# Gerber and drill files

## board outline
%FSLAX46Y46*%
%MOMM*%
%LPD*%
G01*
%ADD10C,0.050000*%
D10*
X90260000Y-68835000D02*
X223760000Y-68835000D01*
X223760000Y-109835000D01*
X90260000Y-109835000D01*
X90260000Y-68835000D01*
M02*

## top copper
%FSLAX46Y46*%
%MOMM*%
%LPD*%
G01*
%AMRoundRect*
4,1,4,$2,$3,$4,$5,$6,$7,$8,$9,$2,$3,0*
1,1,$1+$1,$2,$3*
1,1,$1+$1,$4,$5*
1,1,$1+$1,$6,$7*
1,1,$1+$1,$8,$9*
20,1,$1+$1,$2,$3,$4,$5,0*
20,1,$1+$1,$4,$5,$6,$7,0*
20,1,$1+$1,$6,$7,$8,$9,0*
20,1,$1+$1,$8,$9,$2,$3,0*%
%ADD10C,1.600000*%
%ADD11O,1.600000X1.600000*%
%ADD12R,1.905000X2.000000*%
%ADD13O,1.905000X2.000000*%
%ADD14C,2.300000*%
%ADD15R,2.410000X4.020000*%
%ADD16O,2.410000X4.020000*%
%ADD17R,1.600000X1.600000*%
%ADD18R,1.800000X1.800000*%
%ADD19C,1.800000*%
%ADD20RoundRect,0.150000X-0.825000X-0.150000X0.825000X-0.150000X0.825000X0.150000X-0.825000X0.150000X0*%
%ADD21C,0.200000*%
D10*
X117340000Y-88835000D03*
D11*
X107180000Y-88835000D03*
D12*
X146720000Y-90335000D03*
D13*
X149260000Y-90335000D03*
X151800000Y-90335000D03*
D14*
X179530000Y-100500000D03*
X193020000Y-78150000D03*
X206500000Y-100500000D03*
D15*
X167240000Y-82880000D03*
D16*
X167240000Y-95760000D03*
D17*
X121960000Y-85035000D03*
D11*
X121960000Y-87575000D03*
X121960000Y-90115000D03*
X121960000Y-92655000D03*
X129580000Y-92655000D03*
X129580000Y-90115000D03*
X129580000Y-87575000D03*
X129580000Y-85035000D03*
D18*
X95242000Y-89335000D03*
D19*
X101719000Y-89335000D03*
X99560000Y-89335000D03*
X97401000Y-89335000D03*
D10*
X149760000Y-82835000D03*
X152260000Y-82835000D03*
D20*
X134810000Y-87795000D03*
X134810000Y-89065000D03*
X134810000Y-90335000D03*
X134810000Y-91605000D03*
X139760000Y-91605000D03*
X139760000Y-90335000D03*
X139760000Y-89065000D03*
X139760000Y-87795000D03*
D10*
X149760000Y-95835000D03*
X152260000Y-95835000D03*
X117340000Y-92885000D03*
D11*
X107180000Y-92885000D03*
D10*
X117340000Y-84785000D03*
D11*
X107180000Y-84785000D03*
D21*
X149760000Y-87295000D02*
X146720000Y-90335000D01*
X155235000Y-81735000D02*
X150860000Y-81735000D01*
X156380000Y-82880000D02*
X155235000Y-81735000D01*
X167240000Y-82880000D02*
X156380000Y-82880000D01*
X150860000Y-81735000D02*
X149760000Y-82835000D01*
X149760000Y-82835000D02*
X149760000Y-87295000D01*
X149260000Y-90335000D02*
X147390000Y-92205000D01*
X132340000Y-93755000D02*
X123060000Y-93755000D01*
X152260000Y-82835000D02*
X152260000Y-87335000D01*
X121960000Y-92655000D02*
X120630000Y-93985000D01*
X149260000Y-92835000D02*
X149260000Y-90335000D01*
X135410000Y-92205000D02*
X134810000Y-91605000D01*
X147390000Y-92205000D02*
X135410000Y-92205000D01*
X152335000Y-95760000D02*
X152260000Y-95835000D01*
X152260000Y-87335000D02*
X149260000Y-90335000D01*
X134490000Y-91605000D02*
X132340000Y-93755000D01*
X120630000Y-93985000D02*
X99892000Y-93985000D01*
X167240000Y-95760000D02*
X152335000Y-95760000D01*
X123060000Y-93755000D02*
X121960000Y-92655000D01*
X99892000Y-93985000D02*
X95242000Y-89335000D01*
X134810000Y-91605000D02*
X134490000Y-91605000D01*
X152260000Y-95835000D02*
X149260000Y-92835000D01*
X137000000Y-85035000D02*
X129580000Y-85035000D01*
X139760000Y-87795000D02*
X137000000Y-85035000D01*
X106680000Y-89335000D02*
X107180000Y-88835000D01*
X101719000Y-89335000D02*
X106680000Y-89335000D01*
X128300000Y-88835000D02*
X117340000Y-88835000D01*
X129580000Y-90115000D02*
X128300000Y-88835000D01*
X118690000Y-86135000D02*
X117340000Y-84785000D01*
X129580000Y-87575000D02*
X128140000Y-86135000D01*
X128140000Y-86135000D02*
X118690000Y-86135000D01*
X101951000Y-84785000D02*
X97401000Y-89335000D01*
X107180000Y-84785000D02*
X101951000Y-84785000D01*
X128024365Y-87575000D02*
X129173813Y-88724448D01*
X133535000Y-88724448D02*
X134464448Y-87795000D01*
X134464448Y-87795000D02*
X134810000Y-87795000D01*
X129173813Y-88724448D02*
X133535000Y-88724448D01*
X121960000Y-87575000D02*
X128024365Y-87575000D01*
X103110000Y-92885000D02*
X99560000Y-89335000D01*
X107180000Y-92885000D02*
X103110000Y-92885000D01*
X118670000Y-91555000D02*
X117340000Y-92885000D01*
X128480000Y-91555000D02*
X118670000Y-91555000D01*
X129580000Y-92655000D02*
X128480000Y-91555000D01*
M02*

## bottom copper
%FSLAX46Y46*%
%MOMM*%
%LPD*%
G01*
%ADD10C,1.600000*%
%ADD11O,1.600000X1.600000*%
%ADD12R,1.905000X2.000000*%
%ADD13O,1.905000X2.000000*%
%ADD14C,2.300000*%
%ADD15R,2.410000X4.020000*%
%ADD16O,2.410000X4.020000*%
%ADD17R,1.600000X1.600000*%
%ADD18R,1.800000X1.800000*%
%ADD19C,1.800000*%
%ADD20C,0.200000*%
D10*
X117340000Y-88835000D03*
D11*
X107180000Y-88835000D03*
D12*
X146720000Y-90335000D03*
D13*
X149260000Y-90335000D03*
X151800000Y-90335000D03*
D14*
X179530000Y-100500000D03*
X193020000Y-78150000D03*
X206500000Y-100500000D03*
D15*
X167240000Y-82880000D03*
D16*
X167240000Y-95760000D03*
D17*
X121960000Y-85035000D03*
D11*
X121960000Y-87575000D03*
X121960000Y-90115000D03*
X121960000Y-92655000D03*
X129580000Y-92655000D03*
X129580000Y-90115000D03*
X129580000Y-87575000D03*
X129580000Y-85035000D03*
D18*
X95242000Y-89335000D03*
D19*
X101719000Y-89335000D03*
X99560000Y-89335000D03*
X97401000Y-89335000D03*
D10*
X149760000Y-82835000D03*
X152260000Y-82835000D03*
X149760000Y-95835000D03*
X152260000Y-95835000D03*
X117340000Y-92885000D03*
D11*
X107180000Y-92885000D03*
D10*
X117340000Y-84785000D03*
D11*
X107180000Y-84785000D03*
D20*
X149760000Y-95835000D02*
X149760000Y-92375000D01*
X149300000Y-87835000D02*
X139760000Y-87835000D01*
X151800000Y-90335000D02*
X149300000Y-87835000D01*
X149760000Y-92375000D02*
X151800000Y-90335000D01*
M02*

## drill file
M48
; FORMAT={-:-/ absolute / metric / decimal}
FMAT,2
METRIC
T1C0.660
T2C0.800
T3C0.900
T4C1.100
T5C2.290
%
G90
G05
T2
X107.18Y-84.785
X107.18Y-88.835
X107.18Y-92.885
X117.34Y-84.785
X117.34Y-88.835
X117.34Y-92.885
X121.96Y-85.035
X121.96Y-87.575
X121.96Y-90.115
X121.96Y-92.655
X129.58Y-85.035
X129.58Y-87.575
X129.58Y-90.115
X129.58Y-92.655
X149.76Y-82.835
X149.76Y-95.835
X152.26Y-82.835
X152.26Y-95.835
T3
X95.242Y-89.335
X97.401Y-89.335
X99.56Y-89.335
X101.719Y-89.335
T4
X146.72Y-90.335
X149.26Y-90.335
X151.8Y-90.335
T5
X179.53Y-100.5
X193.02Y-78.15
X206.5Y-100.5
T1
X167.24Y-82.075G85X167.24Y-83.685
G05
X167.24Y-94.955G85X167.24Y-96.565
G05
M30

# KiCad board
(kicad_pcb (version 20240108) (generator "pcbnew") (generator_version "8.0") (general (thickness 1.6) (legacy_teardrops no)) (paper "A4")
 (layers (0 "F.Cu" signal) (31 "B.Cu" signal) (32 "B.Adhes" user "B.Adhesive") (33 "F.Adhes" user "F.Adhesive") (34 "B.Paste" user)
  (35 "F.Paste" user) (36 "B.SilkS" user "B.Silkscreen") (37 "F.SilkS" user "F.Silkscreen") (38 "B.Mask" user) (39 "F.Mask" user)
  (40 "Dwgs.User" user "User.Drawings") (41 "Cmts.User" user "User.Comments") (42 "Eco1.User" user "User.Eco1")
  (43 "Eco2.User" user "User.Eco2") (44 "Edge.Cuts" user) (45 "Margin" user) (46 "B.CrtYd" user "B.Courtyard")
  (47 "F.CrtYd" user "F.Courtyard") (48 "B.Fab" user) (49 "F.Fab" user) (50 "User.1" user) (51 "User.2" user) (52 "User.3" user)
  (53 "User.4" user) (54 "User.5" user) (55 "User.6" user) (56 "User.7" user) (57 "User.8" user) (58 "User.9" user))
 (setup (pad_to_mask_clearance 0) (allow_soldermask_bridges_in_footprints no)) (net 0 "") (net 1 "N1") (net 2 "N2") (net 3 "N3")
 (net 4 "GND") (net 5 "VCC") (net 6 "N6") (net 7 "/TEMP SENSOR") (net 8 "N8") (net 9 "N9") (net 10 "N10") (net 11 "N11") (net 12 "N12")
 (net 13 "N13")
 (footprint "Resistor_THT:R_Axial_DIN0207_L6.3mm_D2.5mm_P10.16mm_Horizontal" (layer "F.Cu") (at 117.34 88.835 180)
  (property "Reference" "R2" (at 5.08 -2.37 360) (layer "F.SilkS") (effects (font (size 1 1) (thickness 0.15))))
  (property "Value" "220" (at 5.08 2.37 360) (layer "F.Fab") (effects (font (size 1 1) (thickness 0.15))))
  (pad "1" thru_hole circle (at 0 0 180) (size 1.6 1.6) (drill 0.8) (layers "*.Cu" "*.Mask") (remove_unused_layers no) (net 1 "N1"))
  (pad "2" thru_hole oval (at 10.16 0 180) (size 1.6 1.6) (drill 0.8) (layers "*.Cu" "*.Mask") (remove_unused_layers no) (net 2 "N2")))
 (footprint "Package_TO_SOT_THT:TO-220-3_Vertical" (layer "F.Cu") (at 146.72 90.335)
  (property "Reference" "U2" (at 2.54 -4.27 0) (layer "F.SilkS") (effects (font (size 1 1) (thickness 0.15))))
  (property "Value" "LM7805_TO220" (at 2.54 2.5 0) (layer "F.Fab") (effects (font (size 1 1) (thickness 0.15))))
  (pad "1" thru_hole rect (at 0 0) (size 1.905 2) (drill 1.1) (layers "*.Cu" "*.Mask") (remove_unused_layers no) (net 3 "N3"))
  (pad "2" thru_hole oval (at 2.54 0) (size 1.905 2) (drill 1.1) (layers "*.Cu" "*.Mask") (remove_unused_layers no) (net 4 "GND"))
  (pad "3" thru_hole oval (at 5.08 0) (size 1.905 2) (drill 1.1) (layers "*.Cu" "*.Mask") (remove_unused_layers no) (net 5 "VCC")))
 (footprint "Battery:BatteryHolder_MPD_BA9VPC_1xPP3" (layer "F.Cu") (at 167.24 82.88)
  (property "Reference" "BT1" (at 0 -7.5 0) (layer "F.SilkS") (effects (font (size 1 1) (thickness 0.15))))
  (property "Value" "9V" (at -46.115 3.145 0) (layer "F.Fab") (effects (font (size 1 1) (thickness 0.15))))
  (pad "" np_thru_hole circle (at 12.29 17.62) (size 2.3 2.3) (drill 2.29) (layers "*.Cu" "*.Mask"))
  (pad "" np_thru_hole circle (at 25.78 -4.73) (size 2.3 2.3) (drill 2.29) (layers "*.Cu" "*.Mask"))
  (pad "" np_thru_hole circle (at 39.26 17.62) (size 2.3 2.3) (drill 2.29) (layers "*.Cu" "*.Mask"))
  (pad "1" thru_hole rect (at 0 0) (size 2.41 4.02) (drill oval 0.66 2.27) (layers "*.Cu" "*.Mask") (remove_unused_layers no) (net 3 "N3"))
  (pad "2" thru_hole oval (at 0 12.88) (size 2.41 4.02) (drill oval 0.66 2.27) (layers "*.Cu" "*.Mask") (remove_unused_layers no)
   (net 4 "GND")))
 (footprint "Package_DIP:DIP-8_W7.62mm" (layer "F.Cu") (at 121.96 85.035)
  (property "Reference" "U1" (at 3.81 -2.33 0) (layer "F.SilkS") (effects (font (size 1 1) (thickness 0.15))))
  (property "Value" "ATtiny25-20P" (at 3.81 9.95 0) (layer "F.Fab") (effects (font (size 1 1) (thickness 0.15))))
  (pad "1" thru_hole rect (at 0 0) (size 1.6 1.6) (drill 0.8) (layers "*.Cu" "*.Mask") (remove_unused_layers no) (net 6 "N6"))
  (pad "2" thru_hole oval (at 0 2.54) (size 1.6 1.6) (drill 0.8) (layers "*.Cu" "*.Mask") (remove_unused_layers no) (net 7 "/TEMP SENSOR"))
  (pad "3" thru_hole oval (at 0 5.08) (size 1.6 1.6) (drill 0.8) (layers "*.Cu" "*.Mask") (remove_unused_layers no) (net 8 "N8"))
  (pad "4" thru_hole oval (at 0 7.62) (size 1.6 1.6) (drill 0.8) (layers "*.Cu" "*.Mask") (remove_unused_layers no) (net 4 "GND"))
  (pad "5" thru_hole oval (at 7.62 7.62) (size 1.6 1.6) (drill 0.8) (layers "*.Cu" "*.Mask") (remove_unused_layers no) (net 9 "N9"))
  (pad "6" thru_hole oval (at 7.62 5.08) (size 1.6 1.6) (drill 0.8) (layers "*.Cu" "*.Mask") (remove_unused_layers no) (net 1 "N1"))
  (pad "7" thru_hole oval (at 7.62 2.54) (size 1.6 1.6) (drill 0.8) (layers "*.Cu" "*.Mask") (remove_unused_layers no) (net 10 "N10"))
  (pad "8" thru_hole oval (at 7.62 0) (size 1.6 1.6) (drill 0.8) (layers "*.Cu" "*.Mask") (remove_unused_layers no) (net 5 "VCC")))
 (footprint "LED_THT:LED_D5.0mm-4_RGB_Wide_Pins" (layer "F.Cu") (at 95.242 89.335)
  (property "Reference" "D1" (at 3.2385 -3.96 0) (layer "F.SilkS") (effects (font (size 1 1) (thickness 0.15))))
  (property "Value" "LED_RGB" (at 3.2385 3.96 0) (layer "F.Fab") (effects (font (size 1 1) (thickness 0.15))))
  (pad "1" thru_hole rect (at 0 0) (size 1.8 1.8) (drill 0.9) (layers "*.Cu" "*.Mask") (remove_unused_layers no) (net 4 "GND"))
  (pad "4" thru_hole circle (at 6.477 0) (size 1.8 1.8) (drill 0.9) (layers "*.Cu" "*.Mask") (remove_unused_layers no) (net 2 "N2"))
  (pad "5" thru_hole circle (at 4.318 0) (size 1.8 1.8) (drill 0.9) (layers "*.Cu" "*.Mask") (remove_unused_layers no) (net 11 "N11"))
  (pad "6" thru_hole circle (at 2.159 0) (size 1.8 1.8) (drill 0.9) (layers "*.Cu" "*.Mask") (remove_unused_layers no) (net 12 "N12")))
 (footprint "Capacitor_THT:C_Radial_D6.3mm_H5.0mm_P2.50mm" (layer "F.Cu") (at 149.76 82.835)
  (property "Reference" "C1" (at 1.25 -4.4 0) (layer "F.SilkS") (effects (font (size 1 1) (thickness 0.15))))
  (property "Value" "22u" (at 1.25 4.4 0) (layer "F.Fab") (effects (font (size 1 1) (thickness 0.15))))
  (pad "1" thru_hole circle (at 0 0) (size 1.6 1.6) (drill 0.8) (layers "*.Cu" "*.Mask") (remove_unused_layers no) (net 3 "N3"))
  (pad "2" thru_hole circle (at 2.5 0) (size 1.6 1.6) (drill 0.8) (layers "*.Cu" "*.Mask") (remove_unused_layers no) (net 4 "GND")))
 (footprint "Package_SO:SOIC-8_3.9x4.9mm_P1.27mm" (layer "F.Cu") (at 137.285 89.7)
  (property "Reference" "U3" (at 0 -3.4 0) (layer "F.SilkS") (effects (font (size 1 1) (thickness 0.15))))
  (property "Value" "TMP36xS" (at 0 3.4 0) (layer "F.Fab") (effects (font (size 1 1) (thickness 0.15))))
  (pad "1" smd roundrect (at -2.475 -1.905) (size 1.95 0.6) (layers "F.Cu" "F.Paste" "F.Mask") (roundrect_rratio 0.25)
   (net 7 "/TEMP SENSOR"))
  (pad "2" smd roundrect (at -2.475 -0.635) (size 1.95 0.6) (layers "F.Cu" "F.Paste" "F.Mask") (roundrect_rratio 0.25))
  (pad "3" smd roundrect (at -2.475 0.635) (size 1.95 0.6) (layers "F.Cu" "F.Paste" "F.Mask") (roundrect_rratio 0.25))
  (pad "4" smd roundrect (at -2.475 1.905) (size 1.95 0.6) (layers "F.Cu" "F.Paste" "F.Mask") (roundrect_rratio 0.25) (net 4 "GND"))
  (pad "5" smd roundrect (at 2.475 1.905) (size 1.95 0.6) (layers "F.Cu" "F.Paste" "F.Mask") (roundrect_rratio 0.25) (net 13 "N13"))
  (pad "6" smd roundrect (at 2.475 0.635) (size 1.95 0.6) (layers "F.Cu" "F.Paste" "F.Mask") (roundrect_rratio 0.25))
  (pad "7" smd roundrect (at 2.475 -0.635) (size 1.95 0.6) (layers "F.Cu" "F.Paste" "F.Mask") (roundrect_rratio 0.25))
  (pad "8" smd roundrect (at 2.475 -1.905) (size 1.95 0.6) (layers "F.Cu" "F.Paste" "F.Mask") (roundrect_rratio 0.25) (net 5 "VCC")))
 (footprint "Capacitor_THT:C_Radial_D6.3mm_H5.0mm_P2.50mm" (layer "F.Cu") (at 149.76 95.835)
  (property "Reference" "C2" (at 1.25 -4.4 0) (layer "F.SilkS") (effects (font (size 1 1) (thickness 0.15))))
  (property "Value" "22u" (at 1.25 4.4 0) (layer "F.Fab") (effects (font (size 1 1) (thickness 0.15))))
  (pad "1" thru_hole circle (at 0 0) (size 1.6 1.6) (drill 0.8) (layers "*.Cu" "*.Mask") (remove_unused_layers no) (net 5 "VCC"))
  (pad "2" thru_hole circle (at 2.5 0) (size 1.6 1.6) (drill 0.8) (layers "*.Cu" "*.Mask") (remove_unused_layers no) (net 4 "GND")))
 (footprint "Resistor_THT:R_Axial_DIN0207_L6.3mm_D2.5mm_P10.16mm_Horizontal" (layer "F.Cu") (at 117.34 92.885 180)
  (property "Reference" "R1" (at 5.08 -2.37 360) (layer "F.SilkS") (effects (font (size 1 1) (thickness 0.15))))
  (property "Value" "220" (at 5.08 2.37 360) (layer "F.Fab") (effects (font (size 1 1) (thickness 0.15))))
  (pad "1" thru_hole circle (at 0 0 180) (size 1.6 1.6) (drill 0.8) (layers "*.Cu" "*.Mask") (remove_unused_layers no) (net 9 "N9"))
  (pad "2" thru_hole oval (at 10.16 0 180) (size 1.6 1.6) (drill 0.8) (layers "*.Cu" "*.Mask") (remove_unused_layers no) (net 11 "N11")))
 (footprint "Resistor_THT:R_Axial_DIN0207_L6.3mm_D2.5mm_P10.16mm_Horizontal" (layer "F.Cu") (at 117.34 84.785 180)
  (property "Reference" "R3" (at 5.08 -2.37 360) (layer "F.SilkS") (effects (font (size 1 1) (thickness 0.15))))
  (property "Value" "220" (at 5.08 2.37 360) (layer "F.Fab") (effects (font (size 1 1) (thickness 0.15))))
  (pad "1" thru_hole circle (at 0 0 180) (size 1.6 1.6) (drill 0.8) (layers "*.Cu" "*.Mask") (remove_unused_layers no) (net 10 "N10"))
  (pad "2" thru_hole oval (at 10.16 0 180) (size 1.6 1.6) (drill 0.8) (layers "*.Cu" "*.Mask") (remove_unused_layers no) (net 12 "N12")))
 (gr_rect (start 90.26 68.835) (end 223.76 109.835) (stroke (width 0.05) (type default)) (fill none) (layer "Edge.Cuts"))
 (segment (start 149.76 87.295) (end 146.72 90.335) (width 0.2) (layer "F.Cu") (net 3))
 (segment (start 155.235 81.735) (end 150.86 81.735) (width 0.2) (layer "F.Cu") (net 3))
 (segment (start 156.38 82.88) (end 155.235 81.735) (width 0.2) (layer "F.Cu") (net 3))
 (segment (start 167.24 82.88) (end 156.38 82.88) (width 0.2) (layer "F.Cu") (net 3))
 (segment (start 150.86 81.735) (end 149.76 82.835) (width 0.2) (layer "F.Cu") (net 3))
 (segment (start 149.76 82.835) (end 149.76 87.295) (width 0.2) (layer "F.Cu") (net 3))
 (segment (start 149.26 90.335) (end 147.39 92.205) (width 0.2) (layer "F.Cu") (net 4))
 (segment (start 132.34 93.755) (end 123.06 93.755) (width 0.2) (layer "F.Cu") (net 4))
 (segment (start 152.26 82.835) (end 152.26 87.335) (width 0.2) (layer "F.Cu") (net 4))
 (segment (start 121.96 92.655) (end 120.63 93.985) (width 0.2) (layer "F.Cu") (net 4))
 (segment (start 149.26 92.835) (end 149.26 90.335) (width 0.2) (layer "F.Cu") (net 4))
 (segment (start 135.41 92.205) (end 134.81 91.605) (width 0.2) (layer "F.Cu") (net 4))
 (segment (start 147.39 92.205) (end 135.41 92.205) (width 0.2) (layer "F.Cu") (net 4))
 (segment (start 152.335 95.76) (end 152.26 95.835) (width 0.2) (layer "F.Cu") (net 4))
 (segment (start 152.26 87.335) (end 149.26 90.335) (width 0.2) (layer "F.Cu") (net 4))
 (segment (start 134.49 91.605) (end 132.34 93.755) (width 0.2) (layer "F.Cu") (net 4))
 (segment (start 120.63 93.985) (end 99.892 93.985) (width 0.2) (layer "F.Cu") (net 4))
 (segment (start 167.24 95.76) (end 152.335 95.76) (width 0.2) (layer "F.Cu") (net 4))
 (segment (start 123.06 93.755) (end 121.96 92.655) (width 0.2) (layer "F.Cu") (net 4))
 (segment (start 99.892 93.985) (end 95.242 89.335) (width 0.2) (layer "F.Cu") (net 4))
 (segment (start 134.81 91.605) (end 134.49 91.605) (width 0.2) (layer "F.Cu") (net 4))
 (segment (start 152.26 95.835) (end 149.26 92.835) (width 0.2) (layer "F.Cu") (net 4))
 (segment (start 137 85.035) (end 129.58 85.035) (width 0.2) (layer "F.Cu") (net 5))
 (segment (start 139.76 87.795) (end 137 85.035) (width 0.2) (layer "F.Cu") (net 5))
 (segment (start 149.76 95.835) (end 149.76 92.375) (width 0.2) (layer "B.Cu") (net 5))
 (segment (start 149.3 87.835) (end 139.76 87.835) (width 0.2) (layer "B.Cu") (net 5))
 (segment (start 151.8 90.335) (end 149.3 87.835) (width 0.2) (layer "B.Cu") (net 5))
 (segment (start 149.76 92.375) (end 151.8 90.335) (width 0.2) (layer "B.Cu") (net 5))
 (segment (start 106.68 89.335) (end 107.18 88.835) (width 0.2) (layer "F.Cu") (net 2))
 (segment (start 101.719 89.335) (end 106.68 89.335) (width 0.2) (layer "F.Cu") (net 2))
 (segment (start 128.3 88.835) (end 117.34 88.835) (width 0.2) (layer "F.Cu") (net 1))
 (segment (start 129.58 90.115) (end 128.3 88.835) (width 0.2) (layer "F.Cu") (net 1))
 (segment (start 118.69 86.135) (end 117.34 84.785) (width 0.2) (layer "F.Cu") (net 10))
 (segment (start 129.58 87.575) (end 128.14 86.135) (width 0.2) (layer "F.Cu") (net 10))
 (segment (start 128.14 86.135) (end 118.69 86.135) (width 0.2) (layer "F.Cu") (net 10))
 (segment (start 101.951 84.785) (end 97.401 89.335) (width 0.2) (layer "F.Cu") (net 12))
 (segment (start 107.18 84.785) (end 101.951 84.785) (width 0.2) (layer "F.Cu") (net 12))
 (segment (start 128.024365 87.575) (end 129.173813 88.724448) (width 0.2) (layer "F.Cu") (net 7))
 (segment (start 133.535 88.724448) (end 134.464448 87.795) (width 0.2) (layer "F.Cu") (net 7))
 (segment (start 134.464448 87.795) (end 134.81 87.795) (width 0.2) (layer "F.Cu") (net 7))
 (segment (start 129.173813 88.724448) (end 133.535 88.724448) (width 0.2) (layer "F.Cu") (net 7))
 (segment (start 121.96 87.575) (end 128.024365 87.575) (width 0.2) (layer "F.Cu") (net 7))
 (segment (start 103.11 92.885) (end 99.56 89.335) (width 0.2) (layer "F.Cu") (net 11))
 (segment (start 107.18 92.885) (end 103.11 92.885) (width 0.2) (layer "F.Cu") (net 11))
 (segment (start 118.67 91.555) (end 117.34 92.885) (width 0.2) (layer "F.Cu") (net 9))
 (segment (start 128.48 91.555) (end 118.67 91.555) (width 0.2) (layer "F.Cu") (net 9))
 (segment (start 129.58 92.655) (end 128.48 91.555) (width 0.2) (layer "F.Cu") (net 9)))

